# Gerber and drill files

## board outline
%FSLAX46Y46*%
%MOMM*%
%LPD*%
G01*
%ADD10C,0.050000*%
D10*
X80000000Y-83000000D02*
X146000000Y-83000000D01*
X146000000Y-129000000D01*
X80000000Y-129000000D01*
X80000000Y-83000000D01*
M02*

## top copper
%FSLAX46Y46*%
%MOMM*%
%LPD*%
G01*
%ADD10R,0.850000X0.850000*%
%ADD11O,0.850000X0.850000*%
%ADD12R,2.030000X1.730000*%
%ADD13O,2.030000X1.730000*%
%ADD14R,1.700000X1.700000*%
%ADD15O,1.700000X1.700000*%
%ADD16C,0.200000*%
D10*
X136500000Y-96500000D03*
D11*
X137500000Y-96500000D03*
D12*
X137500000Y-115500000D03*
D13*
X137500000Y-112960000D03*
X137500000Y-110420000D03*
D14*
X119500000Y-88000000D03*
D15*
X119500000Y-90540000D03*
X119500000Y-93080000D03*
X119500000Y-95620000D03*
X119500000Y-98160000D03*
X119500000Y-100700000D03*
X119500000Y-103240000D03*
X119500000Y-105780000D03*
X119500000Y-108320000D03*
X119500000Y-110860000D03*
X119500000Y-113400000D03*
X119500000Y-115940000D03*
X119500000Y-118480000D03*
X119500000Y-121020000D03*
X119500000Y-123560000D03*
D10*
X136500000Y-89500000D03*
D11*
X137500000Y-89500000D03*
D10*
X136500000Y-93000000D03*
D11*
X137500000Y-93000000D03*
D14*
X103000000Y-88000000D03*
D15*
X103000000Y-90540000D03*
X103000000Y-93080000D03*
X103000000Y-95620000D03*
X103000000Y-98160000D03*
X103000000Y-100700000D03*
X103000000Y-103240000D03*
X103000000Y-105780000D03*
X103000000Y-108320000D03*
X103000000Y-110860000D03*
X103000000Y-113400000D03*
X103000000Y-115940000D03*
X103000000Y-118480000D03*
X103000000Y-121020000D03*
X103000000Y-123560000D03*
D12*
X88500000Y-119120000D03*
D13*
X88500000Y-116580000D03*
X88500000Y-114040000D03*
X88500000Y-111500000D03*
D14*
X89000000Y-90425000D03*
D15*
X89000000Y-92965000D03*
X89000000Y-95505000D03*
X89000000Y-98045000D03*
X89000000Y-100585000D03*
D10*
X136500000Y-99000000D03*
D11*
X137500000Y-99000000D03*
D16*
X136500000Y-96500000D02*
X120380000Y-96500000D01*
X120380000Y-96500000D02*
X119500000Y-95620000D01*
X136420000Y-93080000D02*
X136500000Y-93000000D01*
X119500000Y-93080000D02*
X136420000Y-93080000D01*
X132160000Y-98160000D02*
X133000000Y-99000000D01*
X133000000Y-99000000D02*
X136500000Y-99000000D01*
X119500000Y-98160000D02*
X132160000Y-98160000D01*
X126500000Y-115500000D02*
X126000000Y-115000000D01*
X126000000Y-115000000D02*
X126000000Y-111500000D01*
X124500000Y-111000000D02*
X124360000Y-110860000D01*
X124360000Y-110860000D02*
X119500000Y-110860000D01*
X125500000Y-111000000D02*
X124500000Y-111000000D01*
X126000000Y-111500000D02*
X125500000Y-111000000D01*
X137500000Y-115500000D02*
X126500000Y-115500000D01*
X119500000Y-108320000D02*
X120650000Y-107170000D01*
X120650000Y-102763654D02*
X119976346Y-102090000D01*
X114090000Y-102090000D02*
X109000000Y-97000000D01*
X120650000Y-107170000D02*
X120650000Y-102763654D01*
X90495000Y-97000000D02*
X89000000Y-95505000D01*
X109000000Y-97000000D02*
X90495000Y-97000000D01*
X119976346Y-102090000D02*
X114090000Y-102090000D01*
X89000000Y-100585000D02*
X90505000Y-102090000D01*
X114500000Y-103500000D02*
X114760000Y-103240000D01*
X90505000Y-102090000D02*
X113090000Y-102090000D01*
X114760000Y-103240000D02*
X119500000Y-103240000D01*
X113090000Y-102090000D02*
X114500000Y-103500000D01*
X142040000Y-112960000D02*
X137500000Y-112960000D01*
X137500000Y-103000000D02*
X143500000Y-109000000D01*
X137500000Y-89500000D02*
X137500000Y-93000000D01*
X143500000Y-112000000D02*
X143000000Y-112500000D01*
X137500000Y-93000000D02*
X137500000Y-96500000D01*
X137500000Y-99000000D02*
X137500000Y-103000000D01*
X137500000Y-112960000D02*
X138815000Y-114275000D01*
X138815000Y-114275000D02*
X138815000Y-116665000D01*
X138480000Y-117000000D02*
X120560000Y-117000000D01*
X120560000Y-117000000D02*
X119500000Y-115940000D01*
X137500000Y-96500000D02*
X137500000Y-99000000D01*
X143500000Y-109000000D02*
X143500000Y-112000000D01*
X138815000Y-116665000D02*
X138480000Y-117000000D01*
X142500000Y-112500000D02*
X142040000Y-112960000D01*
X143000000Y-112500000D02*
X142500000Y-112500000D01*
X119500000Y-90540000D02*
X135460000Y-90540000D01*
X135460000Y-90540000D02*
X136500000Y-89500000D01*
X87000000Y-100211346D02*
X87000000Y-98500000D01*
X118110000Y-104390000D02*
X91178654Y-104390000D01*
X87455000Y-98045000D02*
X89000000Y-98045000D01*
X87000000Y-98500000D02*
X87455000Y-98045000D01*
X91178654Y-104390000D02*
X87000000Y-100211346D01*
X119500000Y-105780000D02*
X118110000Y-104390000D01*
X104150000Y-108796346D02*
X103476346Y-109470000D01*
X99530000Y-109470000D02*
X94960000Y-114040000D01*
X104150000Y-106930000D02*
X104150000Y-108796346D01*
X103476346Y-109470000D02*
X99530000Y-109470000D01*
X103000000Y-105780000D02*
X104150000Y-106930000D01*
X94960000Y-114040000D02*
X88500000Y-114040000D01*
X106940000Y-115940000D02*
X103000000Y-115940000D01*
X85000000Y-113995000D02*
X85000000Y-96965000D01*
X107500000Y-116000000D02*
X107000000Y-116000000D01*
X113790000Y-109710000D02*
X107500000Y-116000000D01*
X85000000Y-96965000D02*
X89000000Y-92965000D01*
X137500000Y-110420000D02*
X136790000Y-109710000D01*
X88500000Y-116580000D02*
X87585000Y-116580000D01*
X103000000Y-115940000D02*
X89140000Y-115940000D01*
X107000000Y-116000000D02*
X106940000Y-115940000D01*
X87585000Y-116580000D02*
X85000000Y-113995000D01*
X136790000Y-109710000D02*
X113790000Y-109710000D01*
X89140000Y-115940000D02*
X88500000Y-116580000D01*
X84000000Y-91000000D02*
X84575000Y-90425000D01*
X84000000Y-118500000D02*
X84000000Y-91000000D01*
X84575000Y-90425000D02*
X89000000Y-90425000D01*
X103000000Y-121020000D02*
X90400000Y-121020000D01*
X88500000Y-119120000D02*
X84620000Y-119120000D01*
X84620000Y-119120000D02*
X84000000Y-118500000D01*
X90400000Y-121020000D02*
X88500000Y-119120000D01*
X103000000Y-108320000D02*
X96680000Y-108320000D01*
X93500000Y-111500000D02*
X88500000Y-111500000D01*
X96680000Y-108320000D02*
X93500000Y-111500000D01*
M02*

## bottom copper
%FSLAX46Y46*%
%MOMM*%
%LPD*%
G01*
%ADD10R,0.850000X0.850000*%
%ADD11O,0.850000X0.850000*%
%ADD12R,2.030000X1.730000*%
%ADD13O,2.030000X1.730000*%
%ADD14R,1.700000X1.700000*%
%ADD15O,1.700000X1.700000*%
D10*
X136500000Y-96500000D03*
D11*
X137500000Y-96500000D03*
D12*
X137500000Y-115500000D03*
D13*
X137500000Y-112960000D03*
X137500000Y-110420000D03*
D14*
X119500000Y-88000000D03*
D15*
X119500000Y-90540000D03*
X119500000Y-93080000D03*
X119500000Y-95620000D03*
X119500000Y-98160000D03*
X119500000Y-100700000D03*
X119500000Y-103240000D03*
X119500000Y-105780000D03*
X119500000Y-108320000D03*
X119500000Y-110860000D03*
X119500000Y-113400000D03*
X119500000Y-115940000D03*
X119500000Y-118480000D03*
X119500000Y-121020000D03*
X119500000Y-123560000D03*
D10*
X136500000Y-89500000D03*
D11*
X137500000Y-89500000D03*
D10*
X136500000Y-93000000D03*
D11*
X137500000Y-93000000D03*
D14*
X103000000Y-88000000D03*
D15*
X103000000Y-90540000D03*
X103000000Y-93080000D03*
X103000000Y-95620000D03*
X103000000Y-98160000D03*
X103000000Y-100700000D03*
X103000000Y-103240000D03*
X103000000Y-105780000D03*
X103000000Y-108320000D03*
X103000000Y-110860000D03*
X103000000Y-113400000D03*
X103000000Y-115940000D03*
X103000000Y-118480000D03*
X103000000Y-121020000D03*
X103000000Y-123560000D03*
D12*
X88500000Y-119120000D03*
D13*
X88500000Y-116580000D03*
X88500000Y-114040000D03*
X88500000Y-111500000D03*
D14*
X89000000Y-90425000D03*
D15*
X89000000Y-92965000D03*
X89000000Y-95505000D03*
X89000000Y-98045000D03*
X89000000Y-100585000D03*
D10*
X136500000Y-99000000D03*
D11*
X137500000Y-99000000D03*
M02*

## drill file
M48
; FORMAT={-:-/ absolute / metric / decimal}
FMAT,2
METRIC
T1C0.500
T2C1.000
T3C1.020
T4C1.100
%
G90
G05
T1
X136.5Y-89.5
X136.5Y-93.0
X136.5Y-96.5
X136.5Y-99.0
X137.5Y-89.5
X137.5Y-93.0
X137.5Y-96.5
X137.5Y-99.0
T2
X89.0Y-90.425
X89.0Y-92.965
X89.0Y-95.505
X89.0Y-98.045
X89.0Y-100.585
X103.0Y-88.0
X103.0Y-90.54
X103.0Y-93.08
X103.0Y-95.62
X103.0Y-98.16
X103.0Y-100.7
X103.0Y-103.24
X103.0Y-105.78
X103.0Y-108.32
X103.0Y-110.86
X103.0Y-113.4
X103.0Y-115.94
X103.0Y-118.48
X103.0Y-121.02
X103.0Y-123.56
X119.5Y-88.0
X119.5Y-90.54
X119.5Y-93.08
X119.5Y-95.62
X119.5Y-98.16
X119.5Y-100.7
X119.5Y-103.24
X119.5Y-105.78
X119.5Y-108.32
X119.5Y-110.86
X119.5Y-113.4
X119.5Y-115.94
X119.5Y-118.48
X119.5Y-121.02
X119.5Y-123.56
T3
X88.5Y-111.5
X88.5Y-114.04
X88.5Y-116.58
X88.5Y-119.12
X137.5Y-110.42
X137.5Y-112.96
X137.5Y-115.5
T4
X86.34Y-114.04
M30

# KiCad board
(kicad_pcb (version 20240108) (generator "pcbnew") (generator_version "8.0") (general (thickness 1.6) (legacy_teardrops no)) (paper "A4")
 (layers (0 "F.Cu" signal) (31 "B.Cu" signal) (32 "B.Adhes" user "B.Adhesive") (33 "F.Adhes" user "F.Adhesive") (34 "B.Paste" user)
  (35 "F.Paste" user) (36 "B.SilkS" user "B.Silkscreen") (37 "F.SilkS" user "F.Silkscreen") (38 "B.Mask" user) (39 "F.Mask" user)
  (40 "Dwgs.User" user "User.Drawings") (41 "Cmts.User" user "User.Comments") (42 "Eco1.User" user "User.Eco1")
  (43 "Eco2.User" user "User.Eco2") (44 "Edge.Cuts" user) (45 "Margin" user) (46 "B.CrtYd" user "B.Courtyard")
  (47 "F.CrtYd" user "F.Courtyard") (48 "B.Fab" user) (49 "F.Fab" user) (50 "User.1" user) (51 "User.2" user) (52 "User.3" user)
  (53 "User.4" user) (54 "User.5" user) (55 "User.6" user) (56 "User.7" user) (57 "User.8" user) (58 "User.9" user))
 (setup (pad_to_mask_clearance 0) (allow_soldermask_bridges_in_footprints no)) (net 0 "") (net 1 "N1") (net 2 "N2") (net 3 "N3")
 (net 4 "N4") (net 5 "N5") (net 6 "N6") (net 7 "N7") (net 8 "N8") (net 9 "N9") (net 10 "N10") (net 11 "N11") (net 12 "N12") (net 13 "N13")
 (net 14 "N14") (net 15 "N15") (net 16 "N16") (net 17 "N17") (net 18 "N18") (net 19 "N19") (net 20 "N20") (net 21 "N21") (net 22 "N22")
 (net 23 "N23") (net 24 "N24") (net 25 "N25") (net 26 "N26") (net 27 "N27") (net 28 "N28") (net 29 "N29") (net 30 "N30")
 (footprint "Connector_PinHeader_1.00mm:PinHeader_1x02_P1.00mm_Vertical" (layer "F.Cu") (at 136.5 96.5 90)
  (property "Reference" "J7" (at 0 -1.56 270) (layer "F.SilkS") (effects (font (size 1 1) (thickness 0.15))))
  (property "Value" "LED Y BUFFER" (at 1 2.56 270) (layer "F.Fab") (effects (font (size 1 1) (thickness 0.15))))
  (pad "1" thru_hole rect (at 0 0 90) (size 0.85 0.85) (drill 0.5) (layers "*.Cu" "*.Mask") (remove_unused_layers no) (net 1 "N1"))
  (pad "2" thru_hole oval (at 0 1 90) (size 0.85 0.85) (drill 0.5) (layers "*.Cu" "*.Mask") (remove_unused_layers no) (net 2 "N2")))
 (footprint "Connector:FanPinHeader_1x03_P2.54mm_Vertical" (layer "F.Cu") (at 137.5 115.5 90)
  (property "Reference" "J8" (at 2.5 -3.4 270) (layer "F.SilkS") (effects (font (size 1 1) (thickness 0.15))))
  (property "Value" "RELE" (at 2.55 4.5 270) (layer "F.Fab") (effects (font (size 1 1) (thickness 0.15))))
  (pad "1" thru_hole rect (at 0 0 180) (size 2.03 1.73) (drill 1.02) (layers "*.Cu" "*.Mask") (remove_unused_layers no) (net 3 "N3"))
  (pad "2" thru_hole oval (at 2.54 0 180) (size 2.03 1.73) (drill 1.02) (layers "*.Cu" "*.Mask") (remove_unused_layers no) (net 2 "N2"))
  (pad "3" thru_hole oval (at 5.08 0 180) (size 2.03 1.73) (drill 1.02) (layers "*.Cu" "*.Mask") (remove_unused_layers no) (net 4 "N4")))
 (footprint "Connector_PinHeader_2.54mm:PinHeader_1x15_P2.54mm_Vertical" (layer "F.Cu") (at 119.5 88)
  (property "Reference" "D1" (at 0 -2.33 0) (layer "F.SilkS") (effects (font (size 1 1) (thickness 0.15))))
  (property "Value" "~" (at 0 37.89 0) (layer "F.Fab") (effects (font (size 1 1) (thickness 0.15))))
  (pad "1" thru_hole rect (at 0 0) (size 1.7 1.7) (drill 1) (layers "*.Cu" "*.Mask") (remove_unused_layers no) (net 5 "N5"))
  (pad "2" thru_hole oval (at 0 2.54) (size 1.7 1.7) (drill 1) (layers "*.Cu" "*.Mask") (remove_unused_layers no) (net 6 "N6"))
  (pad "3" thru_hole oval (at 0 5.08) (size 1.7 1.7) (drill 1) (layers "*.Cu" "*.Mask") (remove_unused_layers no) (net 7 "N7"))
  (pad "4" thru_hole oval (at 0 7.62) (size 1.7 1.7) (drill 1) (layers "*.Cu" "*.Mask") (remove_unused_layers no) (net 1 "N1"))
  (pad "5" thru_hole oval (at 0 10.16) (size 1.7 1.7) (drill 1) (layers "*.Cu" "*.Mask") (remove_unused_layers no) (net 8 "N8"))
  (pad "6" thru_hole oval (at 0 12.7) (size 1.7 1.7) (drill 1) (layers "*.Cu" "*.Mask") (remove_unused_layers no) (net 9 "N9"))
  (pad "7" thru_hole oval (at 0 15.24) (size 1.7 1.7) (drill 1) (layers "*.Cu" "*.Mask") (remove_unused_layers no) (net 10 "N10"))
  (pad "8" thru_hole oval (at 0 17.78) (size 1.7 1.7) (drill 1) (layers "*.Cu" "*.Mask") (remove_unused_layers no) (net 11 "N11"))
  (pad "9" thru_hole oval (at 0 20.32) (size 1.7 1.7) (drill 1) (layers "*.Cu" "*.Mask") (remove_unused_layers no) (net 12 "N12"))
  (pad "10" thru_hole oval (at 0 22.86) (size 1.7 1.7) (drill 1) (layers "*.Cu" "*.Mask") (remove_unused_layers no) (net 3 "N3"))
  (pad "11" thru_hole oval (at 0 25.4) (size 1.7 1.7) (drill 1) (layers "*.Cu" "*.Mask") (remove_unused_layers no) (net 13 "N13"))
  (pad "12" thru_hole oval (at 0 27.94) (size 1.7 1.7) (drill 1) (layers "*.Cu" "*.Mask") (remove_unused_layers no) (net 2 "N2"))
  (pad "13" thru_hole oval (at 0 30.48) (size 1.7 1.7) (drill 1) (layers "*.Cu" "*.Mask") (remove_unused_layers no) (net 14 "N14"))
  (pad "14" thru_hole oval (at 0 33.02) (size 1.7 1.7) (drill 1) (layers "*.Cu" "*.Mask") (remove_unused_layers no) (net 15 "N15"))
  (pad "15" thru_hole oval (at 0 35.56) (size 1.7 1.7) (drill 1) (layers "*.Cu" "*.Mask") (remove_unused_layers no) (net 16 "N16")))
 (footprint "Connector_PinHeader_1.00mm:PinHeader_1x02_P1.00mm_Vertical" (layer "F.Cu") (at 136.5 89.5 90)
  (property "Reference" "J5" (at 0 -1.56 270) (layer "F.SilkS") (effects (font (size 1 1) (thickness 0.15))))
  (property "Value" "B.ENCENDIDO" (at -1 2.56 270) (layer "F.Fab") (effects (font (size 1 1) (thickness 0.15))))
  (pad "1" thru_hole rect (at 0 0 90) (size 0.85 0.85) (drill 0.5) (layers "*.Cu" "*.Mask") (remove_unused_layers no) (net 6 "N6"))
  (pad "2" thru_hole oval (at 0 1 90) (size 0.85 0.85) (drill 0.5) (layers "*.Cu" "*.Mask") (remove_unused_layers no) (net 2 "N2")))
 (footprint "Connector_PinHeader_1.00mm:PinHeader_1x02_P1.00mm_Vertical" (layer "F.Cu") (at 136.5 93 90)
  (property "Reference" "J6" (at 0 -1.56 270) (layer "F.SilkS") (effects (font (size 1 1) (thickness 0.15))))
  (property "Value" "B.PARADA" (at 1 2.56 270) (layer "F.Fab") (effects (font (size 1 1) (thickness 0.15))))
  (pad "1" thru_hole rect (at 0 0 90) (size 0.85 0.85) (drill 0.5) (layers "*.Cu" "*.Mask") (remove_unused_layers no) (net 7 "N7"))
  (pad "2" thru_hole oval (at 0 1 90) (size 0.85 0.85) (drill 0.5) (layers "*.Cu" "*.Mask") (remove_unused_layers no) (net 2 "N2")))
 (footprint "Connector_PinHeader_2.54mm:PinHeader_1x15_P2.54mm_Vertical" (layer "F.Cu") (at 103 88)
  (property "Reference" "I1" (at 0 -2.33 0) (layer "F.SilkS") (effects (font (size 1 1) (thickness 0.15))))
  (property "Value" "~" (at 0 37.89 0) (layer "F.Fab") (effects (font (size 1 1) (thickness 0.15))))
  (pad "1" thru_hole rect (at 0 0) (size 1.7 1.7) (drill 1) (layers "*.Cu" "*.Mask") (remove_unused_layers no) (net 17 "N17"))
  (pad "2" thru_hole oval (at 0 2.54) (size 1.7 1.7) (drill 1) (layers "*.Cu" "*.Mask") (remove_unused_layers no) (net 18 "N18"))
  (pad "3" thru_hole oval (at 0 5.08) (size 1.7 1.7) (drill 1) (layers "*.Cu" "*.Mask") (remove_unused_layers no) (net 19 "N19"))
  (pad "4" thru_hole oval (at 0 7.62) (size 1.7 1.7) (drill 1) (layers "*.Cu" "*.Mask") (remove_unused_layers no) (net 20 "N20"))
  (pad "5" thru_hole oval (at 0 10.16) (size 1.7 1.7) (drill 1) (layers "*.Cu" "*.Mask") (remove_unused_layers no) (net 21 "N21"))
  (pad "6" thru_hole oval (at 0 12.7) (size 1.7 1.7) (drill 1) (layers "*.Cu" "*.Mask") (remove_unused_layers no) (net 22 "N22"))
  (pad "7" thru_hole oval (at 0 15.24) (size 1.7 1.7) (drill 1) (layers "*.Cu" "*.Mask") (remove_unused_layers no) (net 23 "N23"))
  (pad "8" thru_hole oval (at 0 17.78) (size 1.7 1.7) (drill 1) (layers "*.Cu" "*.Mask") (remove_unused_layers no) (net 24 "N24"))
  (pad "9" thru_hole oval (at 0 20.32) (size 1.7 1.7) (drill 1) (layers "*.Cu" "*.Mask") (remove_unused_layers no) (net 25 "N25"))
  (pad "10" thru_hole oval (at 0 22.86) (size 1.7 1.7) (drill 1) (layers "*.Cu" "*.Mask") (remove_unused_layers no) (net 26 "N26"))
  (pad "11" thru_hole oval (at 0 25.4) (size 1.7 1.7) (drill 1) (layers "*.Cu" "*.Mask") (remove_unused_layers no) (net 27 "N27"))
  (pad "12" thru_hole oval (at 0 27.94) (size 1.7 1.7) (drill 1) (layers "*.Cu" "*.Mask") (remove_unused_layers no) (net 4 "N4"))
  (pad "13" thru_hole oval (at 0 30.48) (size 1.7 1.7) (drill 1) (layers "*.Cu" "*.Mask") (remove_unused_layers no) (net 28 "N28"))
  (pad "14" thru_hole oval (at 0 33.02) (size 1.7 1.7) (drill 1) (layers "*.Cu" "*.Mask") (remove_unused_layers no) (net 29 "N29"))
  (pad "15" thru_hole oval (at 0 35.56) (size 1.7 1.7) (drill 1) (layers "*.Cu" "*.Mask") (remove_unused_layers no) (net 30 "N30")))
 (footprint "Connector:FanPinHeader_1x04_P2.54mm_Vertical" (layer "F.Cu") (at 88.5 119.12 90)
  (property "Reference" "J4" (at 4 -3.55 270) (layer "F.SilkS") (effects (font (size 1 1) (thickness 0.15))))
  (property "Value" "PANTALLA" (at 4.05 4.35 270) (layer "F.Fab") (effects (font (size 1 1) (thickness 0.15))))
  (pad "" np_thru_hole circle (at 5.08 -2.16 180) (size 1.1 1.1) (drill 1.1) (layers "*.Cu" "*.Mask"))
  (pad "1" thru_hole rect (at 0 0 180) (size 2.03 1.73) (drill 1.02) (layers "*.Cu" "*.Mask") (remove_unused_layers no) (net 29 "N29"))
  (pad "2" thru_hole oval (at 2.54 0 180) (size 2.03 1.73) (drill 1.02) (layers "*.Cu" "*.Mask") (remove_unused_layers no) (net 4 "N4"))
  (pad "3" thru_hole oval (at 5.08 0 180) (size 2.03 1.73) (drill 1.02) (layers "*.Cu" "*.Mask") (remove_unused_layers no) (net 24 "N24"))
  (pad "4" thru_hole oval (at 7.62 0 180) (size 2.03 1.73) (drill 1.02) (layers "*.Cu" "*.Mask") (remove_unused_layers no) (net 25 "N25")))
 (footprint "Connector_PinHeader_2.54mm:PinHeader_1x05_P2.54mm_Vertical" (layer "F.Cu") (at 89 90.425)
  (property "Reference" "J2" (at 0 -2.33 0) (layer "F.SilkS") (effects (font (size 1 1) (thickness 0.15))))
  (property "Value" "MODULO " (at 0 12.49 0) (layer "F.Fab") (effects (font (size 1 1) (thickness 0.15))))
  (pad "1" thru_hole rect (at 0 0) (size 1.7 1.7) (drill 1) (layers "*.Cu" "*.Mask") (remove_unused_layers no) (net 29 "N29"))
  (pad "2" thru_hole oval (at 0 2.54) (size 1.7 1.7) (drill 1) (layers "*.Cu" "*.Mask") (remove_unused_layers no) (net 4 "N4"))
  (pad "3" thru_hole oval (at 0 5.08) (size 1.7 1.7) (drill 1) (layers "*.Cu" "*.Mask") (remove_unused_layers no) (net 12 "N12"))
  (pad "4" thru_hole oval (at 0 7.62) (size 1.7 1.7) (drill 1) (layers "*.Cu" "*.Mask") (remove_unused_layers no) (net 11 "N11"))
  (pad "5" thru_hole oval (at 0 10.16) (size 1.7 1.7) (drill 1) (layers "*.Cu" "*.Mask") (remove_unused_layers no) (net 10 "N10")))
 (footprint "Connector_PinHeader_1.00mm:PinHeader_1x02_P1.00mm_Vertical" (layer "F.Cu") (at 136.5 99 90)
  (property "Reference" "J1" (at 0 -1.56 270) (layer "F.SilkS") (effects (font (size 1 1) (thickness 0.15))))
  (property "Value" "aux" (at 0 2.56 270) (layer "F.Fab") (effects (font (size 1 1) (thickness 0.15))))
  (pad "1" thru_hole rect (at 0 0 90) (size 0.85 0.85) (drill 0.5) (layers "*.Cu" "*.Mask") (remove_unused_layers no) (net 8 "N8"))
  (pad "2" thru_hole oval (at 0 1 90) (size 0.85 0.85) (drill 0.5) (layers "*.Cu" "*.Mask") (remove_unused_layers no) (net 2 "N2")))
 (gr_rect (start 80 83) (end 146 129) (stroke (width 0.05) (type default)) (fill none) (layer "Edge.Cuts"))
 (segment (start 136.5 96.5) (end 120.38 96.5) (width 0.2) (layer "F.Cu") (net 1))
 (segment (start 120.38 96.5) (end 119.5 95.62) (width 0.2) (layer "F.Cu") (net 1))
 (segment (start 136.42 93.08) (end 136.5 93) (width 0.2) (layer "F.Cu") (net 7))
 (segment (start 119.5 93.08) (end 136.42 93.08) (width 0.2) (layer "F.Cu") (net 7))
 (segment (start 132.16 98.16) (end 133 99) (width 0.2) (layer "F.Cu") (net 8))
 (segment (start 133 99) (end 136.5 99) (width 0.2) (layer "F.Cu") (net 8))
 (segment (start 119.5 98.16) (end 132.16 98.16) (width 0.2) (layer "F.Cu") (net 8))
 (segment (start 126.5 115.5) (end 126 115) (width 0.2) (layer "F.Cu") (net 3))
 (segment (start 126 115) (end 126 111.5) (width 0.2) (layer "F.Cu") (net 3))
 (segment (start 124.5 111) (end 124.36 110.86) (width 0.2) (layer "F.Cu") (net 3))
 (segment (start 124.36 110.86) (end 119.5 110.86) (width 0.2) (layer "F.Cu") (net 3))
 (segment (start 125.5 111) (end 124.5 111) (width 0.2) (layer "F.Cu") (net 3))
 (segment (start 126 111.5) (end 125.5 111) (width 0.2) (layer "F.Cu") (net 3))
 (segment (start 137.5 115.5) (end 126.5 115.5) (width 0.2) (layer "F.Cu") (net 3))
 (segment (start 119.5 108.32) (end 120.65 107.17) (width 0.2) (layer "F.Cu") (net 12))
 (segment (start 120.65 102.763654) (end 119.976346 102.09) (width 0.2) (layer "F.Cu") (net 12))
 (segment (start 114.09 102.09) (end 109 97) (width 0.2) (layer "F.Cu") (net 12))
 (segment (start 120.65 107.17) (end 120.65 102.763654) (width 0.2) (layer "F.Cu") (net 12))
 (segment (start 90.495 97) (end 89 95.505) (width 0.2) (layer "F.Cu") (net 12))
 (segment (start 109 97) (end 90.495 97) (width 0.2) (layer "F.Cu") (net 12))
 (segment (start 119.976346 102.09) (end 114.09 102.09) (width 0.2) (layer "F.Cu") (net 12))
 (segment (start 89 100.585) (end 90.505 102.09) (width 0.2) (layer "F.Cu") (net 10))
 (segment (start 114.5 103.5) (end 114.76 103.24) (width 0.2) (layer "F.Cu") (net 10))
 (segment (start 90.505 102.09) (end 113.09 102.09) (width 0.2) (layer "F.Cu") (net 10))
 (segment (start 114.76 103.24) (end 119.5 103.24) (width 0.2) (layer "F.Cu") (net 10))
 (segment (start 113.09 102.09) (end 114.5 103.5) (width 0.2) (layer "F.Cu") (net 10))
 (segment (start 142.04 112.96) (end 137.5 112.96) (width 0.2) (layer "F.Cu") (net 2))
 (segment (start 137.5 103) (end 143.5 109) (width 0.2) (layer "F.Cu") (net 2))
 (segment (start 137.5 89.5) (end 137.5 93) (width 0.2) (layer "F.Cu") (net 2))
 (segment (start 143.5 112) (end 143 112.5) (width 0.2) (layer "F.Cu") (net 2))
 (segment (start 137.5 93) (end 137.5 96.5) (width 0.2) (layer "F.Cu") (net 2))
 (segment (start 137.5 99) (end 137.5 103) (width 0.2) (layer "F.Cu") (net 2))
 (segment (start 137.5 112.96) (end 138.815 114.275) (width 0.2) (layer "F.Cu") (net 2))
 (segment (start 138.815 114.275) (end 138.815 116.665) (width 0.2) (layer "F.Cu") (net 2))
 (segment (start 138.48 117) (end 120.56 117) (width 0.2) (layer "F.Cu") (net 2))
 (segment (start 120.56 117) (end 119.5 115.94) (width 0.2) (layer "F.Cu") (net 2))
 (segment (start 137.5 96.5) (end 137.5 99) (width 0.2) (layer "F.Cu") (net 2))
 (segment (start 143.5 109) (end 143.5 112) (width 0.2) (layer "F.Cu") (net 2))
 (segment (start 138.815 116.665) (end 138.48 117) (width 0.2) (layer "F.Cu") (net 2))
 (segment (start 142.5 112.5) (end 142.04 112.96) (width 0.2) (layer "F.Cu") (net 2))
 (segment (start 143 112.5) (end 142.5 112.5) (width 0.2) (layer "F.Cu") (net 2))
 (segment (start 119.5 90.54) (end 135.46 90.54) (width 0.2) (layer "F.Cu") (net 6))
 (segment (start 135.46 90.54) (end 136.5 89.5) (width 0.2) (layer "F.Cu") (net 6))
 (segment (start 87 100.211346) (end 87 98.5) (width 0.2) (layer "F.Cu") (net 11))
 (segment (start 118.11 104.39) (end 91.178654 104.39) (width 0.2) (layer "F.Cu") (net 11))
 (segment (start 87.455 98.045) (end 89 98.045) (width 0.2) (layer "F.Cu") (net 11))
 (segment (start 87 98.5) (end 87.455 98.045) (width 0.2) (layer "F.Cu") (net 11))
 (segment (start 91.178654 104.39) (end 87 100.211346) (width 0.2) (layer "F.Cu") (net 11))
 (segment (start 119.5 105.78) (end 118.11 104.39) (width 0.2) (layer "F.Cu") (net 11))
 (segment (start 104.15 108.796346) (end 103.476346 109.47) (width 0.2) (layer "F.Cu") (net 24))
 (segment (start 99.53 109.47) (end 94.96 114.04) (width 0.2) (layer "F.Cu") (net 24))
 (segment (start 104.15 106.93) (end 104.15 108.796346) (width 0.2) (layer "F.Cu") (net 24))
 (segment (start 103.476346 109.47) (end 99.53 109.47) (width 0.2) (layer "F.Cu") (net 24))
 (segment (start 103 105.78) (end 104.15 106.93) (width 0.2) (layer "F.Cu") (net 24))
 (segment (start 94.96 114.04) (end 88.5 114.04) (width 0.2) (layer "F.Cu") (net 24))
 (segment (start 106.94 115.94) (end 103 115.94) (width 0.2) (layer "F.Cu") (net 4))
 (segment (start 85 113.995) (end 85 96.965) (width 0.2) (layer "F.Cu") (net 4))
 (segment (start 107.5 116) (end 107 116) (width 0.2) (layer "F.Cu") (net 4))
 (segment (start 113.79 109.71) (end 107.5 116) (width 0.2) (layer "F.Cu") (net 4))
 (segment (start 85 96.965) (end 89 92.965) (width 0.2) (layer "F.Cu") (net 4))
 (segment (start 137.5 110.42) (end 136.79 109.71) (width 0.2) (layer "F.Cu") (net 4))
 (segment (start 88.5 116.58) (end 87.585 116.58) (width 0.2) (layer "F.Cu") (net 4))
 (segment (start 103 115.94) (end 89.14 115.94) (width 0.2) (layer "F.Cu") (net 4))
 (segment (start 107 116) (end 106.94 115.94) (width 0.2) (layer "F.Cu") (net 4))
 (segment (start 87.585 116.58) (end 85 113.995) (width 0.2) (layer "F.Cu") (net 4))
 (segment (start 136.79 109.71) (end 113.79 109.71) (width 0.2) (layer "F.Cu") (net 4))
 (segment (start 89.14 115.94) (end 88.5 116.58) (width 0.2) (layer "F.Cu") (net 4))
 (segment (start 84 91) (end 84.575 90.425) (width 0.2) (layer "F.Cu") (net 29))
 (segment (start 84 118.5) (end 84 91) (width 0.2) (layer "F.Cu") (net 29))
 (segment (start 84.575 90.425) (end 89 90.425) (width 0.2) (layer "F.Cu") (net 29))
 (segment (start 103 121.02) (end 90.4 121.02) (width 0.2) (layer "F.Cu") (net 29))
 (segment (start 88.5 119.12) (end 84.62 119.12) (width 0.2) (layer "F.Cu") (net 29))
 (segment (start 84.62 119.12) (end 84 118.5) (width 0.2) (layer "F.Cu") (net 29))
 (segment (start 90.4 121.02) (end 88.5 119.12) (width 0.2) (layer "F.Cu") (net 29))
 (segment (start 103 108.32) (end 96.68 108.32) (width 0.2) (layer "F.Cu") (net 25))
 (segment (start 93.5 111.5) (end 88.5 111.5) (width 0.2) (layer "F.Cu") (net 25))
 (segment (start 96.68 108.32) (end 93.5 111.5) (width 0.2) (layer "F.Cu") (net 25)))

